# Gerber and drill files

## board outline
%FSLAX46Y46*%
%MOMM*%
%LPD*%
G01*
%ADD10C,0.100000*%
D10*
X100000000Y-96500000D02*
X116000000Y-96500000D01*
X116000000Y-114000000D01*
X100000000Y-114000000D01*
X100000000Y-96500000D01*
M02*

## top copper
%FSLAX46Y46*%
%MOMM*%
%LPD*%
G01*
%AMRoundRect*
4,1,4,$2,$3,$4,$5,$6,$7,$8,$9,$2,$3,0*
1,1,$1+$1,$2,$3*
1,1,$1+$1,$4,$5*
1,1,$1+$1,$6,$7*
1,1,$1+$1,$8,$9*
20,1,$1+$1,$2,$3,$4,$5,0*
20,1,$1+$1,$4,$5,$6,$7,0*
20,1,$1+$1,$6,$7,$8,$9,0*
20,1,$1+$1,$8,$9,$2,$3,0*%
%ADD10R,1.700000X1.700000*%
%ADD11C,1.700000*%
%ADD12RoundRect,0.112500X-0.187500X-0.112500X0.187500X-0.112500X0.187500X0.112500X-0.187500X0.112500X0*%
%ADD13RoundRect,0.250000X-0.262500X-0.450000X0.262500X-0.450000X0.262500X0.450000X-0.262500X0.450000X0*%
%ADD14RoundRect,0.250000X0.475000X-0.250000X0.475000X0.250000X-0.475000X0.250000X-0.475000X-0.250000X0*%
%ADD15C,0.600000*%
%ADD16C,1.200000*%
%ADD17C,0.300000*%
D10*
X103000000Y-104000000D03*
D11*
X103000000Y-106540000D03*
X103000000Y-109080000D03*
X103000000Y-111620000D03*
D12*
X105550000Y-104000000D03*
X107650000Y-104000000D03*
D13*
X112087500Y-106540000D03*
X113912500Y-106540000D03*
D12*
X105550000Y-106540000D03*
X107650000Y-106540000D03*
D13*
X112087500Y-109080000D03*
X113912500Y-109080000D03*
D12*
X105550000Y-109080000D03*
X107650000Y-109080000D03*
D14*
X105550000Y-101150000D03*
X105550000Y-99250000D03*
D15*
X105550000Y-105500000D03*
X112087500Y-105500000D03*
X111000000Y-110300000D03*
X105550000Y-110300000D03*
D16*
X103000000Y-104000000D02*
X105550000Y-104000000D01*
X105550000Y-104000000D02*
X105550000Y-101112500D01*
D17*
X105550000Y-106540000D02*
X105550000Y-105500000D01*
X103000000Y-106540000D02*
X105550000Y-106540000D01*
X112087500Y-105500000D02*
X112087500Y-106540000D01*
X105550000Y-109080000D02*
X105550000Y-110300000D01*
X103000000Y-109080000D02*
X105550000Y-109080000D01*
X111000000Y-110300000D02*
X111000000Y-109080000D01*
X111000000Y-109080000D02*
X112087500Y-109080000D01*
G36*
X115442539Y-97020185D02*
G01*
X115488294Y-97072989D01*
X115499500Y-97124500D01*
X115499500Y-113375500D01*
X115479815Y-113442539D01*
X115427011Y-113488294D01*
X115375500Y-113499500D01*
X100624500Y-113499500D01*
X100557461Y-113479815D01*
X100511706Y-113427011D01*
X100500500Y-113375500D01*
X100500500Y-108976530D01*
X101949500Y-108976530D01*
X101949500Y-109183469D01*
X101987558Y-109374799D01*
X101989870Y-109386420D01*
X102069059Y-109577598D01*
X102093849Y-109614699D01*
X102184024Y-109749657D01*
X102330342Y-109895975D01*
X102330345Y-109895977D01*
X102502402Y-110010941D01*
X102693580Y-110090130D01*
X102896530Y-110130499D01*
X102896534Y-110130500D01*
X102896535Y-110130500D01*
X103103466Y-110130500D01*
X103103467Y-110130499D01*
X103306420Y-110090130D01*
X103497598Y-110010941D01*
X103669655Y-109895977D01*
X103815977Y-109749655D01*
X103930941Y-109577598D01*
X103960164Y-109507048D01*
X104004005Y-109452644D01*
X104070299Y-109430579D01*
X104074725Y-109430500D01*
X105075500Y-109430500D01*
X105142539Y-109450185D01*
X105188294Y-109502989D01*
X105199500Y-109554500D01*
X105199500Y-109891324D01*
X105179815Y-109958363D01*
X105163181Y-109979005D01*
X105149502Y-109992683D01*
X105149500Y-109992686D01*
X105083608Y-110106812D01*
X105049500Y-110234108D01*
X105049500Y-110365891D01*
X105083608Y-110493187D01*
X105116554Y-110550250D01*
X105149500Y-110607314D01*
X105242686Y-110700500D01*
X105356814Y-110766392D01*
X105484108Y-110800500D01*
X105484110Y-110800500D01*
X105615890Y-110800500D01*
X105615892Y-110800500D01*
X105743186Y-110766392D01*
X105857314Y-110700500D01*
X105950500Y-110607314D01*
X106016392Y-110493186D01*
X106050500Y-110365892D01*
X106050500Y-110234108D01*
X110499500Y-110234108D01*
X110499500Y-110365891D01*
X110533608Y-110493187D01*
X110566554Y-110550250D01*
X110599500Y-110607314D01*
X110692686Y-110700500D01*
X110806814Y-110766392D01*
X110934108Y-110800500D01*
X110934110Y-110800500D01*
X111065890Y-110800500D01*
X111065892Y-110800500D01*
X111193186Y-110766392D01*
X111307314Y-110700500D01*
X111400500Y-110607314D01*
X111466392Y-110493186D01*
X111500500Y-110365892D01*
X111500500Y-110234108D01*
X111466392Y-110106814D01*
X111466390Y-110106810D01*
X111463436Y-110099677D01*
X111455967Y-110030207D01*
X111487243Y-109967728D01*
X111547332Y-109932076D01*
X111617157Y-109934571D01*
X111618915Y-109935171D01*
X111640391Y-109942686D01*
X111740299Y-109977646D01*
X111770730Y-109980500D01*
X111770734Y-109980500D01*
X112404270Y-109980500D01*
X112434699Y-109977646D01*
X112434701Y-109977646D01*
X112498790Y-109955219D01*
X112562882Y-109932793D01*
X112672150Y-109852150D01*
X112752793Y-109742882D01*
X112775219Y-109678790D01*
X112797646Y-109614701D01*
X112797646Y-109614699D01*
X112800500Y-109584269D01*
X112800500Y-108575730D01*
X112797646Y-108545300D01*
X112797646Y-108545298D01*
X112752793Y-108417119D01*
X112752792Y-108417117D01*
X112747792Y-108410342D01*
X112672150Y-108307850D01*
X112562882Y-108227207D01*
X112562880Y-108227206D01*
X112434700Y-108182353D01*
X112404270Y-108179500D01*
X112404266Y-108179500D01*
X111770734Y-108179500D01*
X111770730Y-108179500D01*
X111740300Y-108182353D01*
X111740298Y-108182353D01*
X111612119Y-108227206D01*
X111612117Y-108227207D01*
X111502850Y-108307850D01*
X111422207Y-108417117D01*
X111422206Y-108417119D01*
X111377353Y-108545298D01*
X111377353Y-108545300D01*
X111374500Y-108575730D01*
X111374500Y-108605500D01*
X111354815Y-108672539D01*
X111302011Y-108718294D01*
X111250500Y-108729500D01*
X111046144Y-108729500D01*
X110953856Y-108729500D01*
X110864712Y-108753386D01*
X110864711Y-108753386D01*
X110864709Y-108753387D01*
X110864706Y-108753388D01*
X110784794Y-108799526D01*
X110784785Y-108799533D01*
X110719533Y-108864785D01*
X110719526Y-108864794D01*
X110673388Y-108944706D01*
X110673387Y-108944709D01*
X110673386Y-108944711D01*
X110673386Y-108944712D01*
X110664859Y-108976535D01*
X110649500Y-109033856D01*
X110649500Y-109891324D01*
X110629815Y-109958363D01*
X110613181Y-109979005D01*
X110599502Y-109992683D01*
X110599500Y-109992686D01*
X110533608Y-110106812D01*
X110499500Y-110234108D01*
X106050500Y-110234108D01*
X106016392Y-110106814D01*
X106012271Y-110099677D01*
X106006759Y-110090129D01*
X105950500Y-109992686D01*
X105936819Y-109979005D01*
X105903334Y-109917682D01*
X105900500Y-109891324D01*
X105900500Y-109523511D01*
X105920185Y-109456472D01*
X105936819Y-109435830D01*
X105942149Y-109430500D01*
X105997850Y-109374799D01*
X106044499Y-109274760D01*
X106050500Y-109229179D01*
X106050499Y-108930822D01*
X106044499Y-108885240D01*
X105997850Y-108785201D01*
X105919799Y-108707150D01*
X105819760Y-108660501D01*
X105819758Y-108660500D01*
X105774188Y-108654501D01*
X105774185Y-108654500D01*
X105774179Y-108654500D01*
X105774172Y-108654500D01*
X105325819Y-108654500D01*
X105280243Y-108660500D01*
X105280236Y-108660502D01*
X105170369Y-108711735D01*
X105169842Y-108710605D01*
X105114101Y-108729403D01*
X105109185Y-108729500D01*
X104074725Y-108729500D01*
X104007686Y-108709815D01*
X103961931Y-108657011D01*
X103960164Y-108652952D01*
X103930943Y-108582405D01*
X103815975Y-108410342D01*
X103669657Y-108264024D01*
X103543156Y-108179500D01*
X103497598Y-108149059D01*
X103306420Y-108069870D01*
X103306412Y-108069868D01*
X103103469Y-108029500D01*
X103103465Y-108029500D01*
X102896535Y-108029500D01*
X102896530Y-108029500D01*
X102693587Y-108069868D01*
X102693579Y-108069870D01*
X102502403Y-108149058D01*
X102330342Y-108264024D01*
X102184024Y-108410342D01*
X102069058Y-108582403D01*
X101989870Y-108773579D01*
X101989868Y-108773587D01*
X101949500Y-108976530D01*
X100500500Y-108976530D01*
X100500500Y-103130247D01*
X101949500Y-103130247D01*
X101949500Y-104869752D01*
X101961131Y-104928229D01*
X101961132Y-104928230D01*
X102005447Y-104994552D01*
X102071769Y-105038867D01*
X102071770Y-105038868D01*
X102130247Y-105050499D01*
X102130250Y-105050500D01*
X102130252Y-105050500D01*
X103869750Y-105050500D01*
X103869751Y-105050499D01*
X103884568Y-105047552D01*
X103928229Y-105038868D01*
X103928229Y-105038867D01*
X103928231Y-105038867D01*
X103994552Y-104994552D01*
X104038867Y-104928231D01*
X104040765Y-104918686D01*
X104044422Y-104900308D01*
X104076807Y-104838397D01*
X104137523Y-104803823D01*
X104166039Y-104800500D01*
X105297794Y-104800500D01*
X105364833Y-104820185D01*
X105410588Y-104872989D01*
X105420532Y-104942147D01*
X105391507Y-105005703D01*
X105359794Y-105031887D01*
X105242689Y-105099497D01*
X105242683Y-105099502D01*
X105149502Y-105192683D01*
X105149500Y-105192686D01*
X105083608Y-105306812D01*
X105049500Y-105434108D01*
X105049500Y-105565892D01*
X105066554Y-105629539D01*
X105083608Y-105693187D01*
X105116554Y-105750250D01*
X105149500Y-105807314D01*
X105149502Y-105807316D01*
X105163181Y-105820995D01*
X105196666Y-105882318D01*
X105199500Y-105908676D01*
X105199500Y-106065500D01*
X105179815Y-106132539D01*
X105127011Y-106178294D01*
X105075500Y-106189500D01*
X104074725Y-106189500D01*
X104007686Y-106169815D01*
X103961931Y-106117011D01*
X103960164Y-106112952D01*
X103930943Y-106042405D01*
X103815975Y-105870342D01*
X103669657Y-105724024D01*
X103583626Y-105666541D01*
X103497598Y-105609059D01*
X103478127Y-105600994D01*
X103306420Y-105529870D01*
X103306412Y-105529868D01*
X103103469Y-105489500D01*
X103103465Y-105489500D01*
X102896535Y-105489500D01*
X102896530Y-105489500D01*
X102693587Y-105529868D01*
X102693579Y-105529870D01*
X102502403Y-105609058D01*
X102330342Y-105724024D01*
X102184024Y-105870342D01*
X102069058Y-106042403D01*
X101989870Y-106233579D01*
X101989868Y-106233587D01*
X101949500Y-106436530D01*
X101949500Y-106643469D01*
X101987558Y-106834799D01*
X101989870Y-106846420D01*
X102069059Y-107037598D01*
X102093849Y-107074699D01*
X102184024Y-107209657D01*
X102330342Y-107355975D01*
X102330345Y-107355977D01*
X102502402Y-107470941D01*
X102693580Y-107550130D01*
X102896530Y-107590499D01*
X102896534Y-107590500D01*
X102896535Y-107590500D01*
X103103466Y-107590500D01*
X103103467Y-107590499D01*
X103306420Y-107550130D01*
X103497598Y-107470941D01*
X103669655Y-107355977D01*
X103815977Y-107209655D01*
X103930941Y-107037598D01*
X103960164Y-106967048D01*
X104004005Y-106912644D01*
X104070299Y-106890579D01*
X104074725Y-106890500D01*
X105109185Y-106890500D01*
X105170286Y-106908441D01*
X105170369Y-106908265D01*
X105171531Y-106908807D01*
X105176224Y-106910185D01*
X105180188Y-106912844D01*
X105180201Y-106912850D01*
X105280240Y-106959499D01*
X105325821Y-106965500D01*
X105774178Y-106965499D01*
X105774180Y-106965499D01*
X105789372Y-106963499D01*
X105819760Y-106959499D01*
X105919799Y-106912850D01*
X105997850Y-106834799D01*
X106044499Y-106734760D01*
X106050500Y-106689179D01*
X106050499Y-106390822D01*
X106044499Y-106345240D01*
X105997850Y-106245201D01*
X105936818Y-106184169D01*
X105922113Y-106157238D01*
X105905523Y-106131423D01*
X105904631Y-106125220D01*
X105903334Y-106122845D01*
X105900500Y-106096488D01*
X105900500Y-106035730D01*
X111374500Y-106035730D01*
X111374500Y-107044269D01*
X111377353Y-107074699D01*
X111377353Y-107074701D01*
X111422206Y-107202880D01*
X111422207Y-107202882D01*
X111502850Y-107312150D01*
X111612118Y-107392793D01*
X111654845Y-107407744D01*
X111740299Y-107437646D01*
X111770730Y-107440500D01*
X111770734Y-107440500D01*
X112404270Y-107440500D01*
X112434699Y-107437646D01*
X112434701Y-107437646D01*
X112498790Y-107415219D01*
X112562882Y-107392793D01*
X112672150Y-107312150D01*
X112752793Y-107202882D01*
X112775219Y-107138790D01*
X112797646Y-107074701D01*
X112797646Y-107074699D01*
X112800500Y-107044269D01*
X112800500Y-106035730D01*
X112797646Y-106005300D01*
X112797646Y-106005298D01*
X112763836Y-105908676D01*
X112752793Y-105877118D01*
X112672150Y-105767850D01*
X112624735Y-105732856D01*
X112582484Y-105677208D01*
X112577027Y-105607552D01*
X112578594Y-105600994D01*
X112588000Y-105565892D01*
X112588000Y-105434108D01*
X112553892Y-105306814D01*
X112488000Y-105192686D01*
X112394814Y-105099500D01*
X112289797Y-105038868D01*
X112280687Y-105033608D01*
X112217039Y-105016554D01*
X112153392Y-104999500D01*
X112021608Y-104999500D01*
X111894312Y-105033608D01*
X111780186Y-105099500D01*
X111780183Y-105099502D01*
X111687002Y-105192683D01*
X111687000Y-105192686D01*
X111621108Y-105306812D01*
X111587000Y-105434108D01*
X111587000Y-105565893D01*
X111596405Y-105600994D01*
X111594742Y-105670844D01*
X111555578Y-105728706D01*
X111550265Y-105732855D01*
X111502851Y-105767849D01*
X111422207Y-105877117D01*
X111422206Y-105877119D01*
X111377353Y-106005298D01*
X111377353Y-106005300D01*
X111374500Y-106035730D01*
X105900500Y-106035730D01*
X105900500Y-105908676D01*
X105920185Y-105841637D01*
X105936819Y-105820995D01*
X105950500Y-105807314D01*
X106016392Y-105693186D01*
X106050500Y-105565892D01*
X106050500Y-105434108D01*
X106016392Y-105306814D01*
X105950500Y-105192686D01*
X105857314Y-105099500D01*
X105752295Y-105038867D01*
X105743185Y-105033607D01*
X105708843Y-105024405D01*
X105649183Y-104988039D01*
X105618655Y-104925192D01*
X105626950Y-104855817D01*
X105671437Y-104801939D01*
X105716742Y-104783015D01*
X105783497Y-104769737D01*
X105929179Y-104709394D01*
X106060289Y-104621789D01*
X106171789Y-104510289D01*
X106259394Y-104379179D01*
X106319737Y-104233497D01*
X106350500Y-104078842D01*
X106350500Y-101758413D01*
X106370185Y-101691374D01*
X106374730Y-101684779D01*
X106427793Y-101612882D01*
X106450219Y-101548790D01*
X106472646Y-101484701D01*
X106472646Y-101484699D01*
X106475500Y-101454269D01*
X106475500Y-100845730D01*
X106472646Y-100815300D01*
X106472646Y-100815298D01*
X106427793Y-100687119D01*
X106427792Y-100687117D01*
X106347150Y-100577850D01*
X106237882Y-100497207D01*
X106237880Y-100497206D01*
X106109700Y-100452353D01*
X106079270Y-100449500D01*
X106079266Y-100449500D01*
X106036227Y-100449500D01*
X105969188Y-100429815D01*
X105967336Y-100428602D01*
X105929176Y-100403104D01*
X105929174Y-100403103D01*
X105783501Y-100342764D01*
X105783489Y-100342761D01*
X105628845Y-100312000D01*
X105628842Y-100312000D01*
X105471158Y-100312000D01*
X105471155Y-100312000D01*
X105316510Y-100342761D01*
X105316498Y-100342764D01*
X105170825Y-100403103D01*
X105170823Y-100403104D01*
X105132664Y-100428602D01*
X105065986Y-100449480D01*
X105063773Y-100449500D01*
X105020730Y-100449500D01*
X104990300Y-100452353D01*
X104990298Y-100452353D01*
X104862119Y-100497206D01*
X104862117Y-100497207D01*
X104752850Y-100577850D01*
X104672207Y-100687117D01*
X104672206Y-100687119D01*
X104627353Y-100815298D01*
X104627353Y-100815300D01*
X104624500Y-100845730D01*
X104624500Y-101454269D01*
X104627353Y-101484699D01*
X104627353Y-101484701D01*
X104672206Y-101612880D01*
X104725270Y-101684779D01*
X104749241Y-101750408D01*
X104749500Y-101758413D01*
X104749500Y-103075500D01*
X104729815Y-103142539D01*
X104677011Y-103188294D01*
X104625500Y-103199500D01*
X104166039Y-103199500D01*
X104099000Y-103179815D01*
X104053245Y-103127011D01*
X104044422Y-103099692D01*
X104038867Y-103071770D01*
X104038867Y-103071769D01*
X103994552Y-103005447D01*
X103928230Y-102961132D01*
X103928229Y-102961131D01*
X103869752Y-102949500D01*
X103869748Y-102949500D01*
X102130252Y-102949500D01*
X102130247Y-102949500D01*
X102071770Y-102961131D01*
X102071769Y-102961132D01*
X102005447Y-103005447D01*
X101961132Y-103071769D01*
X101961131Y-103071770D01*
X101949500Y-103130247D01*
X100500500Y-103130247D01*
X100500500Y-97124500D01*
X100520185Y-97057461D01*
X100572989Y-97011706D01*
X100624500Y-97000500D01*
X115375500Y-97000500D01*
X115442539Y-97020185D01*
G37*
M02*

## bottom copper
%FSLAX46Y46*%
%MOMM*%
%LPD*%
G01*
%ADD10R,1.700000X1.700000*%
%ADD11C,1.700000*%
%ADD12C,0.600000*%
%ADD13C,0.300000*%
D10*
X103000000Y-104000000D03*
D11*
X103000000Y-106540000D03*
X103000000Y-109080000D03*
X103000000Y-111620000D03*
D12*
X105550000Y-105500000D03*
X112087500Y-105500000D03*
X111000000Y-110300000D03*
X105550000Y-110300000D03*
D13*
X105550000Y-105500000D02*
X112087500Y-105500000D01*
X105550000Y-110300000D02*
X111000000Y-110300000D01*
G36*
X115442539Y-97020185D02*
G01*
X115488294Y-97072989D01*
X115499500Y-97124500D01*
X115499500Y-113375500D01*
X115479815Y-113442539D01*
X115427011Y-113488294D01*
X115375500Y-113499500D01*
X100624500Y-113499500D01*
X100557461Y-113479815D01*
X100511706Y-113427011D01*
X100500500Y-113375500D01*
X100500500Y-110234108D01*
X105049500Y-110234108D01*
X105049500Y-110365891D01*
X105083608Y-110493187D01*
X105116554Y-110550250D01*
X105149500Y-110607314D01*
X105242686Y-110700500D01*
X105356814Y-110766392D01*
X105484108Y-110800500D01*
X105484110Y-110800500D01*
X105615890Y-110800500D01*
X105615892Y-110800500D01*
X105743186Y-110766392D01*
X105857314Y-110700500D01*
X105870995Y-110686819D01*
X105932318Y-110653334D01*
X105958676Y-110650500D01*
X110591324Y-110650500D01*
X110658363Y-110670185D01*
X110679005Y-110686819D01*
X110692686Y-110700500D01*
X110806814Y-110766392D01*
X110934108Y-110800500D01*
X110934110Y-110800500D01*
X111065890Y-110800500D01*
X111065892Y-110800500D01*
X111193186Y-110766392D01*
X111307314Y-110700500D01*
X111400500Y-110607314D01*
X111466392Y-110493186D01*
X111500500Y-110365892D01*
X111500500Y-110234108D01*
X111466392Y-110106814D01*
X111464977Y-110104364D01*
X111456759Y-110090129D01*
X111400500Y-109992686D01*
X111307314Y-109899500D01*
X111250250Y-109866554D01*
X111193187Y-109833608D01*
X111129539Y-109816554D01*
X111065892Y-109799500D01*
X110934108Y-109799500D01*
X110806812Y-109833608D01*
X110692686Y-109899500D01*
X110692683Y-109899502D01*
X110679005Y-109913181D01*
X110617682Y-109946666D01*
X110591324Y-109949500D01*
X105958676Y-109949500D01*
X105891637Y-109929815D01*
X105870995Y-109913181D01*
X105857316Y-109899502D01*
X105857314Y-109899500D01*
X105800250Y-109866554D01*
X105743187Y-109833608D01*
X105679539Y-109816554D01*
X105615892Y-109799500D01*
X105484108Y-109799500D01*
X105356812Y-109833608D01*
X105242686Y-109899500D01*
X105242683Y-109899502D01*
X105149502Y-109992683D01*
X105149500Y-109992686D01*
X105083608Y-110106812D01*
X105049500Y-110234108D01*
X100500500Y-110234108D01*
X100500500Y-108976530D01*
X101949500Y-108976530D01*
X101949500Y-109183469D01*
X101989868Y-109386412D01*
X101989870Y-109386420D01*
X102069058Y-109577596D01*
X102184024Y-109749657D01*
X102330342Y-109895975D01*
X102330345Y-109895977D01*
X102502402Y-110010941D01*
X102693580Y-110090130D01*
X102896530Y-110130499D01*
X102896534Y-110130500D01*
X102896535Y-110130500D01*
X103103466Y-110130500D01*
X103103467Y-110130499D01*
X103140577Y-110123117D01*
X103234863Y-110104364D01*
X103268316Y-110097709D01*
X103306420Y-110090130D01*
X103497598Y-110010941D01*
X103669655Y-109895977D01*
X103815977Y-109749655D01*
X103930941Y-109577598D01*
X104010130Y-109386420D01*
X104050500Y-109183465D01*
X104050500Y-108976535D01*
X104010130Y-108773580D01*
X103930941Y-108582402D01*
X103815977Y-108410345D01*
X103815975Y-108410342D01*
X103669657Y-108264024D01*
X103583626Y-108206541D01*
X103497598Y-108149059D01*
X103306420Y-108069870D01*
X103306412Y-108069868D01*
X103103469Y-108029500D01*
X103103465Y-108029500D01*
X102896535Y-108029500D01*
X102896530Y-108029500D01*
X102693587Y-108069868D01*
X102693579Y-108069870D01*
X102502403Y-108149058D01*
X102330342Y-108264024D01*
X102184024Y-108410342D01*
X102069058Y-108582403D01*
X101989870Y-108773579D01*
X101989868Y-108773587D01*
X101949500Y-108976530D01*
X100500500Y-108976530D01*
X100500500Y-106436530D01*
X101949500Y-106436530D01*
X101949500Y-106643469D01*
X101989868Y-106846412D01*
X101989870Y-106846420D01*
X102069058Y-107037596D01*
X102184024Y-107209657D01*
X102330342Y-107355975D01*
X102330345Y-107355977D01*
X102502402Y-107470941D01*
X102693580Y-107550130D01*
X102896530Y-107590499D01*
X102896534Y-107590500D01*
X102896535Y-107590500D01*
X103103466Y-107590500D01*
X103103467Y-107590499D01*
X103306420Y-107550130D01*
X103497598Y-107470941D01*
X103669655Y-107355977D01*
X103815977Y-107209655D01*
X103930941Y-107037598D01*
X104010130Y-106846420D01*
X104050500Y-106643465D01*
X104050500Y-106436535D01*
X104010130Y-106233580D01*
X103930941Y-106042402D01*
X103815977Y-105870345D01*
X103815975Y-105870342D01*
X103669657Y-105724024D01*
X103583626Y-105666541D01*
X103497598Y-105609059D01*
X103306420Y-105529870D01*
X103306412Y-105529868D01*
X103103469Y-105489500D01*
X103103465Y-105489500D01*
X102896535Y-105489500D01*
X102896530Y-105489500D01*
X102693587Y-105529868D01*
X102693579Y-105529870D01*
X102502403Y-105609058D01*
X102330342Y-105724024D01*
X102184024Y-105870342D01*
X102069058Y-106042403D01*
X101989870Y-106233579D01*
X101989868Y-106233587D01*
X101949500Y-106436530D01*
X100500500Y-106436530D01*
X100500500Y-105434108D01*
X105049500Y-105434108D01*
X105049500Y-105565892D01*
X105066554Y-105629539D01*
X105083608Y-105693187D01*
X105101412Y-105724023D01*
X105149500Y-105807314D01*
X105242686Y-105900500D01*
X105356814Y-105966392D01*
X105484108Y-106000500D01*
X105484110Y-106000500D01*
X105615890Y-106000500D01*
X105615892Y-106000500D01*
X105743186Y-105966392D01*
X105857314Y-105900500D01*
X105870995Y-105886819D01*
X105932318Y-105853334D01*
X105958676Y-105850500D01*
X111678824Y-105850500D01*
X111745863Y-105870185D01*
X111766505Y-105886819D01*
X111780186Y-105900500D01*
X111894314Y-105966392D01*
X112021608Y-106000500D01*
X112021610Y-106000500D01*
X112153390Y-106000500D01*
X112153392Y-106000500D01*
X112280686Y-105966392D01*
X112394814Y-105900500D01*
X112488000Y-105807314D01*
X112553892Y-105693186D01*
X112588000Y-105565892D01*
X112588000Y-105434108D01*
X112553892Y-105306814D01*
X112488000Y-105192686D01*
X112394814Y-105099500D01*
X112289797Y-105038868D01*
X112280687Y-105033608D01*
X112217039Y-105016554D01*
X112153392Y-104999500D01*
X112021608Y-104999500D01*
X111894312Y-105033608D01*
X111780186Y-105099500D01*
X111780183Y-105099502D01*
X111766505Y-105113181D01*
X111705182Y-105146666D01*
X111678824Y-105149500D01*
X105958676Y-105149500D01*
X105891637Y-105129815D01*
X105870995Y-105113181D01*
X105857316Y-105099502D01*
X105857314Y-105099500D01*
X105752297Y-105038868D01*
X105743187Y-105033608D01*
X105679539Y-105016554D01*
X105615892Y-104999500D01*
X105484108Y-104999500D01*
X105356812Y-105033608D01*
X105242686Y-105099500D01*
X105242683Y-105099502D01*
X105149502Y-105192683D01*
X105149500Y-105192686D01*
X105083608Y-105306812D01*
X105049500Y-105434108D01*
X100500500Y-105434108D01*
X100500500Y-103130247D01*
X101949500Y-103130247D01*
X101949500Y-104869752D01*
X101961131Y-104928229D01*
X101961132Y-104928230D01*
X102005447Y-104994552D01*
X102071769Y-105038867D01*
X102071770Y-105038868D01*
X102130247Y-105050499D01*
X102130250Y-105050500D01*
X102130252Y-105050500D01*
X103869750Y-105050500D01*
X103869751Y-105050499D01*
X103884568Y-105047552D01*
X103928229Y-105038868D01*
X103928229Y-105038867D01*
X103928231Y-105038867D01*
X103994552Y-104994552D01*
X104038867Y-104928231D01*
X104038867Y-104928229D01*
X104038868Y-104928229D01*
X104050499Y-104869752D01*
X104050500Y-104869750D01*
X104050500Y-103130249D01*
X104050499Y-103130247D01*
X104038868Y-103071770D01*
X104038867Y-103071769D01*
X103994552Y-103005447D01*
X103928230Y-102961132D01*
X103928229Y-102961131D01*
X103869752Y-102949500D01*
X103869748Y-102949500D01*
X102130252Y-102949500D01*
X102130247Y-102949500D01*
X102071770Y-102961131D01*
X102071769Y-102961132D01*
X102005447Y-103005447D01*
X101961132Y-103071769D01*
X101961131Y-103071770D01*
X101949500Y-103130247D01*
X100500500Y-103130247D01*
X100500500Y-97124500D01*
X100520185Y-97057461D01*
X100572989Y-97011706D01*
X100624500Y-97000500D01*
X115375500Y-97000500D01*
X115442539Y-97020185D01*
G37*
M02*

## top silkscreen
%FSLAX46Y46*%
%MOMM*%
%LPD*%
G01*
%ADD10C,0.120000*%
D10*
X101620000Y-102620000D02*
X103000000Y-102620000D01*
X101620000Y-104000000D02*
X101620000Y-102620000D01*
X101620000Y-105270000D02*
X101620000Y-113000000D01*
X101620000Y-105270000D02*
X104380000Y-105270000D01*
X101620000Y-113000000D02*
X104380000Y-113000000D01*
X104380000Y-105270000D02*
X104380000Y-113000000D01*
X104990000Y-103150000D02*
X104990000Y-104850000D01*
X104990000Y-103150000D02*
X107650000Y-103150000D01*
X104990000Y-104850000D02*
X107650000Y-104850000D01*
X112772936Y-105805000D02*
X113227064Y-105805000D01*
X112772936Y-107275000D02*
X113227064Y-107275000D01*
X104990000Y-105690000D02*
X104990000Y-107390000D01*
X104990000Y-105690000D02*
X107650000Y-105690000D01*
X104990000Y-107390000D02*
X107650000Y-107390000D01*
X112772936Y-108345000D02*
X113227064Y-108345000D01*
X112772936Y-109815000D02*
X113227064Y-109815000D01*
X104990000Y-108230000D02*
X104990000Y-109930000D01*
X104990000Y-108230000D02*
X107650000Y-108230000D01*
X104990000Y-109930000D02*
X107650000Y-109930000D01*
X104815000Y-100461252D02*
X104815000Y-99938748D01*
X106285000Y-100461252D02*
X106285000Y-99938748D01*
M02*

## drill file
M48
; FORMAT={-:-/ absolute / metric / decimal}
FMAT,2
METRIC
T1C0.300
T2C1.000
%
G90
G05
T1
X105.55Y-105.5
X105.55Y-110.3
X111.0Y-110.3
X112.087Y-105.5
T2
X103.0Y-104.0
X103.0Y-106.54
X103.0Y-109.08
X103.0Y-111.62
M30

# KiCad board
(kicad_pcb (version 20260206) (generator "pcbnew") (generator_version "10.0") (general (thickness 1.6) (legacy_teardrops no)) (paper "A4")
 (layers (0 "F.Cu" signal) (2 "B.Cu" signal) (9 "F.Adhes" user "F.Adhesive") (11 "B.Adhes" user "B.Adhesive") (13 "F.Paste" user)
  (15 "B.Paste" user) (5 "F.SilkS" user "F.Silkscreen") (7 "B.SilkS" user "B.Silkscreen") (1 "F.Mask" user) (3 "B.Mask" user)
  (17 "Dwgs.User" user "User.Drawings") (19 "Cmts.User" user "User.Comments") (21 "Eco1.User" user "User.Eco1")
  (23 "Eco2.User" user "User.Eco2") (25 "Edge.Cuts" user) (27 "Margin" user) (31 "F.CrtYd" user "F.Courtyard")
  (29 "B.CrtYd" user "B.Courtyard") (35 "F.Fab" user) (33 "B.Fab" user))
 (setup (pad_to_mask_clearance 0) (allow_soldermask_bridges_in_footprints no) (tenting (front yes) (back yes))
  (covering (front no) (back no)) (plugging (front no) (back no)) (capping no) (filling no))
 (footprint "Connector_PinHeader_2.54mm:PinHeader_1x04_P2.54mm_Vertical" (layer "F.Cu") (at 103 104)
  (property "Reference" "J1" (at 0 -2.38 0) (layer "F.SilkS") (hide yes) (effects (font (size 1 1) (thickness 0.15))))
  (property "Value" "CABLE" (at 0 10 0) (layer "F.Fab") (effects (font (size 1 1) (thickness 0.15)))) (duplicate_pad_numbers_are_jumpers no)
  (fp_line (start -1.38 -1.38) (end 0 -1.38) (stroke (width 0.12) (type solid)) (layer "F.SilkS"))
  (fp_line (start -1.38 0) (end -1.38 -1.38) (stroke (width 0.12) (type solid)) (layer "F.SilkS"))
  (fp_line (start -1.38 1.27) (end -1.38 9) (stroke (width 0.12) (type solid)) (layer "F.SilkS"))
  (fp_line (start -1.38 1.27) (end 1.38 1.27) (stroke (width 0.12) (type solid)) (layer "F.SilkS"))
  (fp_line (start -1.38 9) (end 1.38 9) (stroke (width 0.12) (type solid)) (layer "F.SilkS"))
  (fp_line (start 1.38 1.27) (end 1.38 9) (stroke (width 0.12) (type solid)) (layer "F.SilkS"))
  (pad "1" thru_hole rect (at 0 0) (size 1.7 1.7) (drill 1) (layers "*.Cu" "*.Mask") (remove_unused_layers no) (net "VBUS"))
  (pad "2" thru_hole circle (at 0 2.54) (size 1.7 1.7) (drill 1) (layers "*.Cu" "*.Mask") (remove_unused_layers no) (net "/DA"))
  (pad "3" thru_hole circle (at 0 5.08) (size 1.7 1.7) (drill 1) (layers "*.Cu" "*.Mask") (remove_unused_layers no) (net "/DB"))
  (pad "4" thru_hole circle (at 0 7.62) (size 1.7 1.7) (drill 1) (layers "*.Cu" "*.Mask") (remove_unused_layers no) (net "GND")))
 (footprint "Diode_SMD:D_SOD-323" (layer "F.Cu") (at 106.6 104)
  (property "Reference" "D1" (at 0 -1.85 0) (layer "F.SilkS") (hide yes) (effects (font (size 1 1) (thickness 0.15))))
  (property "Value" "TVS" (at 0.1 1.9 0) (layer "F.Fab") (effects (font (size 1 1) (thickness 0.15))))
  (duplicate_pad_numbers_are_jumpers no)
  (fp_line (start -1.61 -0.85) (end -1.61 0.85) (stroke (width 0.12) (type solid)) (layer "F.SilkS"))
  (fp_line (start -1.61 -0.85) (end 1.05 -0.85) (stroke (width 0.12) (type solid)) (layer "F.SilkS"))
  (fp_line (start -1.61 0.85) (end 1.05 0.85) (stroke (width 0.12) (type solid)) (layer "F.SilkS"))
  (pad "1" smd roundrect (at -1.05 0) (size 0.6 0.45) (layers "F.Cu" "F.Mask" "F.Paste") (roundrect_rratio 0.25) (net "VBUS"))
  (pad "2" smd roundrect (at 1.05 0) (size 0.6 0.45) (layers "F.Cu" "F.Mask" "F.Paste") (roundrect_rratio 0.25) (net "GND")))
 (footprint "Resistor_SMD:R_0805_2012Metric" (layer "F.Cu") (at 113 106.54)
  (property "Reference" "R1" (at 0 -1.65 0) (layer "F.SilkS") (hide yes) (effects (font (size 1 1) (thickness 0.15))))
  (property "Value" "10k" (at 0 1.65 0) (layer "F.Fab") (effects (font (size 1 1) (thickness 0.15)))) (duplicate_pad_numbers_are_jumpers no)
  (fp_line (start -0.227064 -0.735) (end 0.227064 -0.735) (stroke (width 0.12) (type solid)) (layer "F.SilkS"))
  (fp_line (start -0.227064 0.735) (end 0.227064 0.735) (stroke (width 0.12) (type solid)) (layer "F.SilkS"))
  (pad "1" smd roundrect (at -0.9125 0) (size 1.025 1.4) (layers "F.Cu" "F.Mask" "F.Paste") (roundrect_rratio 0.243902) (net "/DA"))
  (pad "2" smd roundrect (at 0.9125 0) (size 1.025 1.4) (layers "F.Cu" "F.Mask" "F.Paste") (roundrect_rratio 0.243902) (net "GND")))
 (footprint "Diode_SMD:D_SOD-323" (layer "F.Cu") (at 106.6 106.54)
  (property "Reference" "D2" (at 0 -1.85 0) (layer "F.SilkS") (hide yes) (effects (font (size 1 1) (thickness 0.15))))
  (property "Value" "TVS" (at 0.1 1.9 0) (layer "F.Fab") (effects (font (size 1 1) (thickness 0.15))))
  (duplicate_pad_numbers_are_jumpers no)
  (fp_line (start -1.61 -0.85) (end -1.61 0.85) (stroke (width 0.12) (type solid)) (layer "F.SilkS"))
  (fp_line (start -1.61 -0.85) (end 1.05 -0.85) (stroke (width 0.12) (type solid)) (layer "F.SilkS"))
  (fp_line (start -1.61 0.85) (end 1.05 0.85) (stroke (width 0.12) (type solid)) (layer "F.SilkS"))
  (pad "1" smd roundrect (at -1.05 0) (size 0.6 0.45) (layers "F.Cu" "F.Mask" "F.Paste") (roundrect_rratio 0.25) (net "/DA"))
  (pad "2" smd roundrect (at 1.05 0) (size 0.6 0.45) (layers "F.Cu" "F.Mask" "F.Paste") (roundrect_rratio 0.25) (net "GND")))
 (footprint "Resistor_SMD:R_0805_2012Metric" (layer "F.Cu") (at 113 109.08)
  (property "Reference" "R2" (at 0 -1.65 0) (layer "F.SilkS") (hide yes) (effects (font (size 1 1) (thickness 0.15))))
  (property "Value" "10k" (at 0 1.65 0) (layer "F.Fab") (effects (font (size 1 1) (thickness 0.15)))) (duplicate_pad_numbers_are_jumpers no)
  (fp_line (start -0.227064 -0.735) (end 0.227064 -0.735) (stroke (width 0.12) (type solid)) (layer "F.SilkS"))
  (fp_line (start -0.227064 0.735) (end 0.227064 0.735) (stroke (width 0.12) (type solid)) (layer "F.SilkS"))
  (pad "1" smd roundrect (at -0.9125 0) (size 1.025 1.4) (layers "F.Cu" "F.Mask" "F.Paste") (roundrect_rratio 0.243902) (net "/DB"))
  (pad "2" smd roundrect (at 0.9125 0) (size 1.025 1.4) (layers "F.Cu" "F.Mask" "F.Paste") (roundrect_rratio 0.243902) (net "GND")))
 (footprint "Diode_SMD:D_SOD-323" (layer "F.Cu") (at 106.6 109.08)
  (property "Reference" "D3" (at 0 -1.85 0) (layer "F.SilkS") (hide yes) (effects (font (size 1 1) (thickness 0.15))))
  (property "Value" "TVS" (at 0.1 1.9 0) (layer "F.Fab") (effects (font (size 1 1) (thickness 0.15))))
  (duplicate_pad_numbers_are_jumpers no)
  (fp_line (start -1.61 -0.85) (end -1.61 0.85) (stroke (width 0.12) (type solid)) (layer "F.SilkS"))
  (fp_line (start -1.61 -0.85) (end 1.05 -0.85) (stroke (width 0.12) (type solid)) (layer "F.SilkS"))
  (fp_line (start -1.61 0.85) (end 1.05 0.85) (stroke (width 0.12) (type solid)) (layer "F.SilkS"))
  (pad "1" smd roundrect (at -1.05 0) (size 0.6 0.45) (layers "F.Cu" "F.Mask" "F.Paste") (roundrect_rratio 0.25) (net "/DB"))
  (pad "2" smd roundrect (at 1.05 0) (size 0.6 0.45) (layers "F.Cu" "F.Mask" "F.Paste") (roundrect_rratio 0.25) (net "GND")))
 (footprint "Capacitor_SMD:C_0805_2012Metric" (layer "F.Cu") (at 105.55 100.2 90)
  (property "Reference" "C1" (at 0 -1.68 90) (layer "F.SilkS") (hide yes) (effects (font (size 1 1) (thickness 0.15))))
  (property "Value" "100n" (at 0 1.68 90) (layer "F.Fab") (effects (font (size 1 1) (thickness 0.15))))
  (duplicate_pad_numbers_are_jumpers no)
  (fp_line (start -0.261252 -0.735) (end 0.261252 -0.735) (stroke (width 0.12) (type solid)) (layer "F.SilkS"))
  (fp_line (start -0.261252 0.735) (end 0.261252 0.735) (stroke (width 0.12) (type solid)) (layer "F.SilkS"))
  (pad "1" smd roundrect (at -0.95 0 90) (size 1 1.45) (layers "F.Cu" "F.Mask" "F.Paste") (roundrect_rratio 0.25) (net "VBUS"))
  (pad "2" smd roundrect (at 0.95 0 90) (size 1 1.45) (layers "F.Cu" "F.Mask" "F.Paste") (roundrect_rratio 0.25) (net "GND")))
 (gr_rect (start 100 96.5) (end 116 114) (stroke (width 0.1) (type default)) (fill no) (layer "Edge.Cuts"))
 (segment (start 103 104) (end 105.55 104) (width 1.2) (layer "F.Cu") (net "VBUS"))
 (segment (start 105.55 104) (end 105.55 101.1125) (width 1.2) (layer "F.Cu") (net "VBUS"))
 (segment (start 105.55 106.54) (end 105.55 105.5) (width 0.3) (layer "F.Cu") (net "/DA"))
 (segment (start 103 106.54) (end 105.55 106.54) (width 0.3) (layer "F.Cu") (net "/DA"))
 (segment (start 112.0875 105.5) (end 112.0875 106.54) (width 0.3) (layer "F.Cu") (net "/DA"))
 (via (at 105.55 105.5) (size 0.6) (drill 0.3) (layers "F.Cu" "B.Cu") (capping no) (covering (front no) (back no))
  (plugging (front no) (back no)) (filling no) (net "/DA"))
 (via (at 112.0875 105.5) (size 0.6) (drill 0.3) (layers "F.Cu" "B.Cu") (capping no) (covering (front no) (back no))
  (plugging (front no) (back no)) (filling no) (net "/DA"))
 (segment (start 105.55 105.5) (end 112.0875 105.5) (width 0.3) (layer "B.Cu") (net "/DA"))
 (segment (start 105.55 109.08) (end 105.55 110.3) (width 0.3) (layer "F.Cu") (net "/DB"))
 (segment (start 103 109.08) (end 105.55 109.08) (width 0.3) (layer "F.Cu") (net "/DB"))
 (segment (start 111 110.3) (end 111 109.08) (width 0.3) (layer "F.Cu") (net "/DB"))
 (segment (start 111 109.08) (end 112.0875 109.08) (width 0.3) (layer "F.Cu") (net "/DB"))
 (via (at 111 110.3) (size 0.6) (drill 0.3) (layers "F.Cu" "B.Cu") (capping no) (covering (front no) (back no))
  (plugging (front no) (back no)) (filling no) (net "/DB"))
 (via (at 105.55 110.3) (size 0.6) (drill 0.3) (layers "F.Cu" "B.Cu") (capping no) (covering (front no) (back no))
  (plugging (front no) (back no)) (filling no) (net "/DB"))
 (segment (start 105.55 110.3) (end 111 110.3) (width 0.3) (layer "B.Cu") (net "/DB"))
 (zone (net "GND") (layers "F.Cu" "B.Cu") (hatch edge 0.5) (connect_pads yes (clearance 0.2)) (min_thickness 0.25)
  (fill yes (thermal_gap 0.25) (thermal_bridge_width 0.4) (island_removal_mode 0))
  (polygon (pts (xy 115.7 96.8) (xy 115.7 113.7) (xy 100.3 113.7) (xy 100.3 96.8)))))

